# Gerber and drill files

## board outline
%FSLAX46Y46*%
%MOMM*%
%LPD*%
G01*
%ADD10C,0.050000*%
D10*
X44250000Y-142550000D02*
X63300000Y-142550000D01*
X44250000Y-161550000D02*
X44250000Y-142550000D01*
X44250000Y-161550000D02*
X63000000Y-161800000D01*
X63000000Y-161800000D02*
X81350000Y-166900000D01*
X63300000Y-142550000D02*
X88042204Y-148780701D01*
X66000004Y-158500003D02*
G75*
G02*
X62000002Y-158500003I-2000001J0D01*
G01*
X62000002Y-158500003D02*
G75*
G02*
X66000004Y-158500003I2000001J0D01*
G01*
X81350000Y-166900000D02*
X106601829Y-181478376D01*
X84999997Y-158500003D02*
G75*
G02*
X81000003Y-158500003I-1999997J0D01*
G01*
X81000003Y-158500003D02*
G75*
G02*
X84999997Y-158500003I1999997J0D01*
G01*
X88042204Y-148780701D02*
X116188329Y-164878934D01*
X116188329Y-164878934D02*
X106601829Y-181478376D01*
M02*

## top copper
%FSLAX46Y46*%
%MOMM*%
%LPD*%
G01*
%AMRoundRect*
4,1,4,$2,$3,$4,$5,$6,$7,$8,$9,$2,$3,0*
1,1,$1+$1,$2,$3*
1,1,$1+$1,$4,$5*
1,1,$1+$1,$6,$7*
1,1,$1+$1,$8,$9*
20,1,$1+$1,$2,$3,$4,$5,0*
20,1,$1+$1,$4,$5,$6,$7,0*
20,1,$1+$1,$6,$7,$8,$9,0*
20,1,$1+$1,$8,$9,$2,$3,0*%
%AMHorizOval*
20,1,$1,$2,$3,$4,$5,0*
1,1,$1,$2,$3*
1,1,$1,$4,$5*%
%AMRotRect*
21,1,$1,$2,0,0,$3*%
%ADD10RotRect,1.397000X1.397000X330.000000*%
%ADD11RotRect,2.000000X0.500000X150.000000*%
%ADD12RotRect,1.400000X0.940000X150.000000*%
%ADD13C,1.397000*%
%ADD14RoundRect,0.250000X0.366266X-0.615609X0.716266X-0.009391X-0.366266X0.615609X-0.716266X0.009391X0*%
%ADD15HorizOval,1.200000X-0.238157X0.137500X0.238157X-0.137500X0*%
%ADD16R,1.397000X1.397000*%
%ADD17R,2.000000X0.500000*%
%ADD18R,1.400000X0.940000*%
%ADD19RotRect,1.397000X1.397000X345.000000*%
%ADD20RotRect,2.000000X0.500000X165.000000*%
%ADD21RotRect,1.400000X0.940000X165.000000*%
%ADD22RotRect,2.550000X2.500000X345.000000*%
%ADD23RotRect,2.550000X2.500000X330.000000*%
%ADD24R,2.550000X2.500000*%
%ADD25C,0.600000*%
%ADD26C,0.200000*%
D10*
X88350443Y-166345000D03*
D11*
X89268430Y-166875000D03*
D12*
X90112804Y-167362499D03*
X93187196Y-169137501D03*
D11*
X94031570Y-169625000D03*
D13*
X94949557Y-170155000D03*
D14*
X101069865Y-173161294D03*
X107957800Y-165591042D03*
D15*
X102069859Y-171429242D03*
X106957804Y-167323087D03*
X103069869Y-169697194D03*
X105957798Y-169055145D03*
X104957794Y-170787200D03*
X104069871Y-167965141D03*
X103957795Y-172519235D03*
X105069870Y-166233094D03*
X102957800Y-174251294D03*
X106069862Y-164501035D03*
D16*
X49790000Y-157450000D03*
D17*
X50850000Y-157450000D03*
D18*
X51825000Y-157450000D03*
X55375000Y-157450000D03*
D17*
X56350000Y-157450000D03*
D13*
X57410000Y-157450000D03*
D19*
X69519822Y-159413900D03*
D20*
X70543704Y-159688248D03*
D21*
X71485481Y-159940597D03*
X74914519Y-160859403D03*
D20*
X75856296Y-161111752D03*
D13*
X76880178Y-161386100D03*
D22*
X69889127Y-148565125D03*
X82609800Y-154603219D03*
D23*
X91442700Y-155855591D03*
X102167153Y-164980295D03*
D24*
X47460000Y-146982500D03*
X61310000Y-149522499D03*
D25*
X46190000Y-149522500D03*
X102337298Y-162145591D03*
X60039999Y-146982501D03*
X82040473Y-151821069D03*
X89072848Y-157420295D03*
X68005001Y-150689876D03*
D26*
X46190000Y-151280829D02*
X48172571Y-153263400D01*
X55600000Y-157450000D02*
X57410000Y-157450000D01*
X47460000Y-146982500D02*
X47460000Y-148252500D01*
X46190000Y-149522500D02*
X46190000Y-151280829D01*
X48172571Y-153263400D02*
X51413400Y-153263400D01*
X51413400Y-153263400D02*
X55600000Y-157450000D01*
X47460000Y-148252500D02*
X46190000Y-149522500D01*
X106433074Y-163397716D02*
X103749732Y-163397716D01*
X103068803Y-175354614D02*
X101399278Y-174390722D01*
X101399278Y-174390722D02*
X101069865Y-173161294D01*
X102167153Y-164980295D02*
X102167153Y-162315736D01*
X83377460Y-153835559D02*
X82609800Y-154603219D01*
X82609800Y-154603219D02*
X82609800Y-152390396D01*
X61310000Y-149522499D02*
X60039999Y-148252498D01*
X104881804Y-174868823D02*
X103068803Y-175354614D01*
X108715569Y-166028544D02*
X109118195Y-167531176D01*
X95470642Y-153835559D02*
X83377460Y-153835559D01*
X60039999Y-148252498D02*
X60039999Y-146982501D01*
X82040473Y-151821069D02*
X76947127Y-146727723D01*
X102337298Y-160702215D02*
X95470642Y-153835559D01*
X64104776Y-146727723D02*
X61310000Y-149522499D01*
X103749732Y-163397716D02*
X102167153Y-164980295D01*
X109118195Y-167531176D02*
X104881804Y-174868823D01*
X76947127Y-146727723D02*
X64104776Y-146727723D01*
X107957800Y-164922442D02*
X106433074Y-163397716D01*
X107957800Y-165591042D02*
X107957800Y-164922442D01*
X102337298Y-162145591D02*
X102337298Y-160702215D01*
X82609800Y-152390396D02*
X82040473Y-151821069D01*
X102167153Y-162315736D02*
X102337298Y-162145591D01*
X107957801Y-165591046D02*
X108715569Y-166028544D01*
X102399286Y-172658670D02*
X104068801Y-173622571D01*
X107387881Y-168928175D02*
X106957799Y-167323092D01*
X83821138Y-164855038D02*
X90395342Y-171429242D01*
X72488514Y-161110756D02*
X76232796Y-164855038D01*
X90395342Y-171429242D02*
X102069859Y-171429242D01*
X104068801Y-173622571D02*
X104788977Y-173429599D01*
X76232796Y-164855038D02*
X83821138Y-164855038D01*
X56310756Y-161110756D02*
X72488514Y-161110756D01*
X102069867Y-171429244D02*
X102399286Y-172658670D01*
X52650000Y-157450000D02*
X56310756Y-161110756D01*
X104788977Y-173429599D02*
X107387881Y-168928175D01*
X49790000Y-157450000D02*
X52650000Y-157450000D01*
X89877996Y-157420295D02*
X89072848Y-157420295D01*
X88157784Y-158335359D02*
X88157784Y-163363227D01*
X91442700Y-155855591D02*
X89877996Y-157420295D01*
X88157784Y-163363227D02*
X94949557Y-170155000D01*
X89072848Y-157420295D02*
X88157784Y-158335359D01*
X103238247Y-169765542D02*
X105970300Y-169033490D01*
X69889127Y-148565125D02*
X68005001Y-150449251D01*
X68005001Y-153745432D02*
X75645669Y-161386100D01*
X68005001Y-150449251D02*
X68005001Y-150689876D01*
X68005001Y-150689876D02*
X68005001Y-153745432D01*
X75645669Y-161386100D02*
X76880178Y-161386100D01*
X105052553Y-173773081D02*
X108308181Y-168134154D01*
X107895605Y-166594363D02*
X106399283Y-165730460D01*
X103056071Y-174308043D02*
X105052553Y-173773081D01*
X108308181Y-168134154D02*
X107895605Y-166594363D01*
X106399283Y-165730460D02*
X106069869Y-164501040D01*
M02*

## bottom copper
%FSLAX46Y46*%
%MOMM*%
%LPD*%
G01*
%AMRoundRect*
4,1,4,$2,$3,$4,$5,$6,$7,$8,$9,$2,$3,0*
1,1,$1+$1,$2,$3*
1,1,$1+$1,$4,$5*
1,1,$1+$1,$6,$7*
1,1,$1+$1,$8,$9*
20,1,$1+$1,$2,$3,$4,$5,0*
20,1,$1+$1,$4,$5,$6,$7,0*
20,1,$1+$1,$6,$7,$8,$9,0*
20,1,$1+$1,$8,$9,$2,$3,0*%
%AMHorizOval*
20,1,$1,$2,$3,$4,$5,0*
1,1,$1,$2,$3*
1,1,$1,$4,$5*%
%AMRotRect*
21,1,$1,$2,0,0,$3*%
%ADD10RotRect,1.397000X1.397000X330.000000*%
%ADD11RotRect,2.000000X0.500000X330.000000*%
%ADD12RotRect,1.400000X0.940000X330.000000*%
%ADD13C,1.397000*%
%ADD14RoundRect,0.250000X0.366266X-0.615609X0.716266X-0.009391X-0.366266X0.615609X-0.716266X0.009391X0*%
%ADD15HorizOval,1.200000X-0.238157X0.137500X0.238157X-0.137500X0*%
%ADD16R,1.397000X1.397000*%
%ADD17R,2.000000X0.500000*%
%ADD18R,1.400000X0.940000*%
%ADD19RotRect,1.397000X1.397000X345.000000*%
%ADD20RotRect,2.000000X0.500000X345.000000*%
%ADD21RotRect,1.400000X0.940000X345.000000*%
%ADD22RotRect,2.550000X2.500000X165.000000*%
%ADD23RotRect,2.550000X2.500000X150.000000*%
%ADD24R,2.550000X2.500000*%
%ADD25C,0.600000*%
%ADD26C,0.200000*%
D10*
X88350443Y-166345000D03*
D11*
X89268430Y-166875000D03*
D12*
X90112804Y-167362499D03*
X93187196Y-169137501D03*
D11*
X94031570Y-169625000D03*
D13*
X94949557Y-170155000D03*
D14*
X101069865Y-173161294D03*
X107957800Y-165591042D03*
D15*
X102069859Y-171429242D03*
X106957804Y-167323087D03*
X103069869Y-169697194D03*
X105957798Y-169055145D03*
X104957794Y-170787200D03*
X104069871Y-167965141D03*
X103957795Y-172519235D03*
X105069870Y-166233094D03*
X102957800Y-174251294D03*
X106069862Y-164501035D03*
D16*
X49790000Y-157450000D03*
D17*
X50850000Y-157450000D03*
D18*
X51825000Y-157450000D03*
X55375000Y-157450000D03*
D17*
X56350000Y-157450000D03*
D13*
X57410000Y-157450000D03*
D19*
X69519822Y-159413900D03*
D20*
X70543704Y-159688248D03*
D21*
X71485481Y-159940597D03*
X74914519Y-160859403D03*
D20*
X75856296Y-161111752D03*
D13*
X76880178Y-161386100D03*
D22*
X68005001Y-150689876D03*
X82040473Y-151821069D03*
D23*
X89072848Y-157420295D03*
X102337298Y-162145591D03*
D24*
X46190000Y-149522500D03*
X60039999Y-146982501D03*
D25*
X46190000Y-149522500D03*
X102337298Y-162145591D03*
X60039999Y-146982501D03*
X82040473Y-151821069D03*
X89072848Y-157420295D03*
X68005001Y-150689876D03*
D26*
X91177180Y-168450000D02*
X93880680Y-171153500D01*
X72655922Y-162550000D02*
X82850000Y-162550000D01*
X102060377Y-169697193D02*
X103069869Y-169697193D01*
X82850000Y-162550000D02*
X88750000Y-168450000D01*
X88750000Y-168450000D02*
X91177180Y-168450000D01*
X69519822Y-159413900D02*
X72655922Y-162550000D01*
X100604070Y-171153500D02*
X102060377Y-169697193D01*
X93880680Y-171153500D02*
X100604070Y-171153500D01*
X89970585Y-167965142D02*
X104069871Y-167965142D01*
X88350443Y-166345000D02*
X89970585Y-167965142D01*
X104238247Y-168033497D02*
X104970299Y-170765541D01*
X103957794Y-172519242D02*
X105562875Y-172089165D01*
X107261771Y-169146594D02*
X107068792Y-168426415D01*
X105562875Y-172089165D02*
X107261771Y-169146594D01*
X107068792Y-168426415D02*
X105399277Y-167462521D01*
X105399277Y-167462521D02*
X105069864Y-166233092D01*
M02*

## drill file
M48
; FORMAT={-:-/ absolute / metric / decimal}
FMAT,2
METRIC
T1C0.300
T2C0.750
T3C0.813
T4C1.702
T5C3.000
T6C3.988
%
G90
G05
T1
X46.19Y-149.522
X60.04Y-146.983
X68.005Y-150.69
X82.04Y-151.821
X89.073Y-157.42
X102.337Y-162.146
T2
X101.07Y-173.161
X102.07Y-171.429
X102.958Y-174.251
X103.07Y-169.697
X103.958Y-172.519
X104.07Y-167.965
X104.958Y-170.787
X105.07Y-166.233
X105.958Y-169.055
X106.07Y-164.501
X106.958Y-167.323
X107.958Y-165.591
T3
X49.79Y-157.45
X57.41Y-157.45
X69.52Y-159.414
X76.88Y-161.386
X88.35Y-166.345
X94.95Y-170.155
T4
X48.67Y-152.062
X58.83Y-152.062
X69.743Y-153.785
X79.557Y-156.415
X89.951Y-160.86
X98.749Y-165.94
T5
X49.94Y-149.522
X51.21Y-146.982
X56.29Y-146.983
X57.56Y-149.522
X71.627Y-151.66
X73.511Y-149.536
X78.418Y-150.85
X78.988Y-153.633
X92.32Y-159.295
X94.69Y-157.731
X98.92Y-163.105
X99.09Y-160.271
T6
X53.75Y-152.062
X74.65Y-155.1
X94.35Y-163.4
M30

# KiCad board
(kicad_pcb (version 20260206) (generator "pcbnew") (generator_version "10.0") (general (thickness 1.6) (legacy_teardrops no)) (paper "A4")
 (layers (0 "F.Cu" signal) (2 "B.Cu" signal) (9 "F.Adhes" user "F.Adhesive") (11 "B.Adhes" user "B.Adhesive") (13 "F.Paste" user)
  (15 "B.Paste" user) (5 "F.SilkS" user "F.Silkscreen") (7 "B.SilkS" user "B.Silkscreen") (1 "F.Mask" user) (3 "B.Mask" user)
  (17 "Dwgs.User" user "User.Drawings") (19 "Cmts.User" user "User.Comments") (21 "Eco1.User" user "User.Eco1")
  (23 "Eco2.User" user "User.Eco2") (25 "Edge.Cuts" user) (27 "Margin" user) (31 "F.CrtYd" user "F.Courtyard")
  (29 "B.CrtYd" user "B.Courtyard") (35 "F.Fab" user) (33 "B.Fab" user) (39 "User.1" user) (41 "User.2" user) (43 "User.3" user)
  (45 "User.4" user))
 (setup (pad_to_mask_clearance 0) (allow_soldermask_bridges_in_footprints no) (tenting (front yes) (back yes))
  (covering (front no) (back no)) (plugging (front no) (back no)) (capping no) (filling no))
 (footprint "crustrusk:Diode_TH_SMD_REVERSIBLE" (layer "F.Cu") (at 91.65 168.25 -30)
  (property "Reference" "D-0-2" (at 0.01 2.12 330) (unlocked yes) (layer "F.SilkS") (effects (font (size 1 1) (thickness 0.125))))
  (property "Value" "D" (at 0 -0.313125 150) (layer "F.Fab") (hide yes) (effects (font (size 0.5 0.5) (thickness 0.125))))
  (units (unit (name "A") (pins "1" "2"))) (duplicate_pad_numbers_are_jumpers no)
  (pad "1" thru_hole rect (at -3.81 0 330) (size 1.397 1.397) (drill 0.8128) (layers "*.Cu" "*.Mask") (remove_unused_layers no)
   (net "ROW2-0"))
  (pad "1" smd rect (at -2.75 0 150) (size 2 0.5) (layers "F.Cu") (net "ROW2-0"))
  (pad "1" smd rect (at -2.75 0 330) (size 2 0.5) (layers "B.Cu") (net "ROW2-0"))
  (pad "1" smd rect (at -1.775001 0 150) (size 1.4 0.94) (layers "F.Cu" "F.Mask" "F.Paste") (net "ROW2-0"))
  (pad "1" smd rect (at -1.775001 0 330) (size 1.4 0.94) (layers "B.Cu" "B.Mask" "B.Paste") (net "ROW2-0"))
  (pad "2" smd rect (at 1.775001 0 150) (size 1.4 0.94) (layers "F.Cu" "F.Mask" "F.Paste") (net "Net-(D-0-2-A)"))
  (pad "2" smd rect (at 1.775001 0 330) (size 1.4 0.94) (layers "B.Cu" "B.Mask" "B.Paste") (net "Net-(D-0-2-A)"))
  (pad "2" smd rect (at 2.75 0 150) (size 2 0.5) (layers "F.Cu") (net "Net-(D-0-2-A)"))
  (pad "2" smd rect (at 2.75 0 330) (size 2 0.5) (layers "B.Cu") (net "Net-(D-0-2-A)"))
  (pad "2" thru_hole circle (at 3.81 0 330) (size 1.397 1.397) (drill 0.8128) (layers "*.Cu" "*.Mask") (remove_unused_layers no)
   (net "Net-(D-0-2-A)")))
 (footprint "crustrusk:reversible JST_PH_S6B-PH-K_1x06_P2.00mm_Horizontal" (layer "F.Cu") (at 101.069865 173.161294 60)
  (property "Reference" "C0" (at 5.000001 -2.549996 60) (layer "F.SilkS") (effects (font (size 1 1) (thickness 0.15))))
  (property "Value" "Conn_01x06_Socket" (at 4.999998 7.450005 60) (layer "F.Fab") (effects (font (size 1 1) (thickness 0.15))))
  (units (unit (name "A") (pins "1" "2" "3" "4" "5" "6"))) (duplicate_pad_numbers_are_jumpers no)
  (pad "1" thru_hole roundrect (at 0 0 60) (size 1.2 1.75) (drill 0.75) (layers "*.Cu" "*.Mask") (remove_unused_layers no)
   (roundrect_rratio 0.208333) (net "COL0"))
  (pad "1" thru_hole roundrect (at 9.999998 2.180001 60) (size 1.2 1.75) (drill 0.75) (layers "*.Cu" "*.Mask") (remove_unused_layers no)
   (roundrect_rratio 0.208333) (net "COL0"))
  (pad "2" thru_hole oval (at 1.999998 -0.000006 60) (size 1.2 1.75) (drill 0.75) (layers "*.Cu" "*.Mask") (remove_unused_layers no)
   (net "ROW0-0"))
  (pad "2" thru_hole oval (at 8.000005 2.180001 60) (size 1.2 1.75) (drill 0.75) (layers "*.Cu" "*.Mask") (remove_unused_layers no)
   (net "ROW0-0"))
  (pad "3" thru_hole oval (at 4.000001 0.000004 60) (size 1.2 1.75) (drill 0.75) (layers "*.Cu" "*.Mask") (remove_unused_layers no)
   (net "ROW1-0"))
  (pad "3" thru_hole oval (at 5.999996 2.18 60) (size 1.2 1.75) (drill 0.75) (layers "*.Cu" "*.Mask") (remove_unused_layers no)
   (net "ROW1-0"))
  (pad "4" thru_hole oval (at 3.99999 2.179998 60) (size 1.2 1.75) (drill 0.75) (layers "*.Cu" "*.Mask") (remove_unused_layers no)
   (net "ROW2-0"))
  (pad "4" thru_hole oval (at 6.000003 0.000005 60) (size 1.2 1.75) (drill 0.75) (layers "*.Cu" "*.Mask") (remove_unused_layers no)
   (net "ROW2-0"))
  (pad "5" thru_hole oval (at 2.000004 2.179991 60) (size 1.2 1.75) (drill 0.75) (layers "*.Cu" "*.Mask") (remove_unused_layers no)
   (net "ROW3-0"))
  (pad "5" thru_hole oval (at 8 0.000006 60) (size 1.2 1.75) (drill 0.75) (layers "*.Cu" "*.Mask") (remove_unused_layers no) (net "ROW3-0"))
  (pad "6" thru_hole oval (at 0 2.18 60) (size 1.2 1.75) (drill 0.75) (layers "*.Cu" "*.Mask") (remove_unused_layers no) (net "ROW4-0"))
  (pad "6" thru_hole oval (at 10.000003 -0.000005 60) (size 1.2 1.75) (drill 0.75) (layers "*.Cu" "*.Mask") (remove_unused_layers no)
   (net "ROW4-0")))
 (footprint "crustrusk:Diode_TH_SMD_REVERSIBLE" (layer "F.Cu") (at 53.6 157.45)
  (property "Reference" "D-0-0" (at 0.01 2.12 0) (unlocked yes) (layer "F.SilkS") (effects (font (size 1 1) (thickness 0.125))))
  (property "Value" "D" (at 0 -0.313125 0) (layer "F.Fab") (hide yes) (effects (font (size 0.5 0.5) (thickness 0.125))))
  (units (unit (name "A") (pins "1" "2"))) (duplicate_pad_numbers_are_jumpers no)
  (pad "1" thru_hole rect (at -3.81 0) (size 1.397 1.397) (drill 0.8128) (layers "*.Cu" "*.Mask") (remove_unused_layers no) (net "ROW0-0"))
  (pad "1" smd rect (at -2.75 0 180) (size 2 0.5) (layers "F.Cu") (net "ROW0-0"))
  (pad "1" smd rect (at -2.75 0) (size 2 0.5) (layers "B.Cu") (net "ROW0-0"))
  (pad "1" smd rect (at -1.775 0 180) (size 1.4 0.94) (layers "F.Cu" "F.Mask" "F.Paste") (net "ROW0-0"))
  (pad "1" smd rect (at -1.775 0) (size 1.4 0.94) (layers "B.Cu" "B.Mask" "B.Paste") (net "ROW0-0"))
  (pad "2" smd rect (at 1.775 0 180) (size 1.4 0.94) (layers "F.Cu" "F.Mask" "F.Paste") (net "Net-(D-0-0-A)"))
  (pad "2" smd rect (at 1.775 0) (size 1.4 0.94) (layers "B.Cu" "B.Mask" "B.Paste") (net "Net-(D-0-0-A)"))
  (pad "2" smd rect (at 2.75 0 180) (size 2 0.5) (layers "F.Cu") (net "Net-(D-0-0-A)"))
  (pad "2" smd rect (at 2.75 0) (size 2 0.5) (layers "B.Cu") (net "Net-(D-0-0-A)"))
  (pad "2" thru_hole circle (at 3.81 0) (size 1.397 1.397) (drill 0.8128) (layers "*.Cu" "*.Mask") (remove_unused_layers no)
   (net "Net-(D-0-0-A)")))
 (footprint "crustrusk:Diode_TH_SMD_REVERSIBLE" (layer "F.Cu") (at 73.2 160.4 -15)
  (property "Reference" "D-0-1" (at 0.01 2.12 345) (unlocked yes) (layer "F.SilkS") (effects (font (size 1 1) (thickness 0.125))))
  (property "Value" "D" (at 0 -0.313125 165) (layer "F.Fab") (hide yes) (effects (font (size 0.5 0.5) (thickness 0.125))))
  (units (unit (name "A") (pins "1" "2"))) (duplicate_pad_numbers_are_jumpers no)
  (pad "1" thru_hole rect (at -3.81 0.000001 345) (size 1.397 1.397) (drill 0.8128) (layers "*.Cu" "*.Mask") (remove_unused_layers no)
   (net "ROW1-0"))
  (pad "1" smd rect (at -2.75 0 165) (size 2 0.5) (layers "F.Cu") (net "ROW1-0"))
  (pad "1" smd rect (at -2.75 0 345) (size 2 0.5) (layers "B.Cu") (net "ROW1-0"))
  (pad "1" smd rect (at -1.775 0.000001 165) (size 1.4 0.94) (layers "F.Cu" "F.Mask" "F.Paste") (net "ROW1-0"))
  (pad "1" smd rect (at -1.775 0.000001 345) (size 1.4 0.94) (layers "B.Cu" "B.Mask" "B.Paste") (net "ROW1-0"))
  (pad "2" smd rect (at 1.775 -0.000001 165) (size 1.4 0.94) (layers "F.Cu" "F.Mask" "F.Paste") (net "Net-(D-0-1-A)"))
  (pad "2" smd rect (at 1.775 -0.000001 345) (size 1.4 0.94) (layers "B.Cu" "B.Mask" "B.Paste") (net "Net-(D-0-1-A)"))
  (pad "2" smd rect (at 2.75 0 165) (size 2 0.5) (layers "F.Cu") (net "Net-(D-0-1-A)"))
  (pad "2" smd rect (at 2.75 0 345) (size 2 0.5) (layers "B.Cu") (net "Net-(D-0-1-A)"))
  (pad "2" thru_hole circle (at 3.81 -0.000001 345) (size 1.397 1.397) (drill 0.8128) (layers "*.Cu" "*.Mask") (remove_unused_layers no)
   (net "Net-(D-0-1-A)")))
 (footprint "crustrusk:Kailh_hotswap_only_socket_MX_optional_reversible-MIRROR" (layer "B.Cu") (at 74.65 155.1 165)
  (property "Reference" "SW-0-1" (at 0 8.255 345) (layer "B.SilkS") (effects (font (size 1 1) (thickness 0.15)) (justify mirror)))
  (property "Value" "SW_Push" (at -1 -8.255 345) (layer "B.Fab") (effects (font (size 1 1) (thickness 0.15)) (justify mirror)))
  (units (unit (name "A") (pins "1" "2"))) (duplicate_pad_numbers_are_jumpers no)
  (pad "" np_thru_hole circle (at -5.08 0 165) (size 1.7018 1.7018) (drill 1.7018) (layers "*.Cu" "*.Mask"))
  (pad "" np_thru_hole circle (at -3.81 2.54 345) (size 3 3) (drill 3) (layers "*.Cu" "*.Mask"))
  (pad "" np_thru_hole circle (at -2.54 5.079998 165) (size 3 3) (drill 3) (layers "*.Cu" "*.Mask"))
  (pad "" np_thru_hole circle (at 0 0 165) (size 3.9878 3.9878) (drill 3.9878) (layers "*.Cu" "*.Mask"))
  (pad "" np_thru_hole circle (at 2.540002 5.080001 345) (size 3 3) (drill 3) (layers "*.Cu" "*.Mask"))
  (pad "" np_thru_hole circle (at 3.81 2.54 165) (size 3 3) (drill 3) (layers "*.Cu" "*.Mask"))
  (pad "" np_thru_hole circle (at 5.08 0 165) (size 1.7018 1.7018) (drill 1.7018) (layers "*.Cu" "*.Mask"))
  (pad "1" smd rect (at 6.29 5.08 345) (size 2.55 2.5) (layers "F.Cu" "F.Mask" "F.Paste") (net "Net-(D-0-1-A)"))
  (pad "1" smd rect (at 7.56 2.54 165) (size 2.55 2.5) (layers "B.Cu" "B.Mask" "B.Paste") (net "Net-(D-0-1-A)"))
  (pad "2" smd rect (at -7.56 2.540001 345) (size 2.55 2.5) (layers "F.Cu" "F.Mask" "F.Paste") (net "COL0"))
  (pad "2" smd rect (at -6.289999 5.079999 165) (size 2.55 2.5) (layers "B.Cu" "B.Mask" "B.Paste") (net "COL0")))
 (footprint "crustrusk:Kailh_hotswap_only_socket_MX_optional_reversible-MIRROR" (layer "B.Cu") (at 94.35 163.4 150)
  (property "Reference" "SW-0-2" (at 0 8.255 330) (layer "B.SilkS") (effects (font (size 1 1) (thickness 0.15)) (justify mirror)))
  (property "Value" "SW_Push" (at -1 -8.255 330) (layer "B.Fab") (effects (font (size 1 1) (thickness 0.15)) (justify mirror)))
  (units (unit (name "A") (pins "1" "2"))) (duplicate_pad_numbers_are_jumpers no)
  (pad "" np_thru_hole circle (at -5.08 0 150) (size 1.7018 1.7018) (drill 1.7018) (layers "*.Cu" "*.Mask"))
  (pad "" np_thru_hole circle (at -3.81 2.540001 330) (size 3 3) (drill 3) (layers "*.Cu" "*.Mask"))
  (pad "" np_thru_hole circle (at -2.540001 5.079998 150) (size 3 3) (drill 3) (layers "*.Cu" "*.Mask"))
  (pad "" np_thru_hole circle (at 0 0 150) (size 3.9878 3.9878) (drill 3.9878) (layers "*.Cu" "*.Mask"))
  (pad "" np_thru_hole circle (at 2.540002 5.080001 330) (size 3 3) (drill 3) (layers "*.Cu" "*.Mask"))
  (pad "" np_thru_hole circle (at 3.81 2.54 150) (size 3 3) (drill 3) (layers "*.Cu" "*.Mask"))
  (pad "" np_thru_hole circle (at 5.08 0 150) (size 1.7018 1.7018) (drill 1.7018) (layers "*.Cu" "*.Mask"))
  (pad "1" smd rect (at 6.29 5.08 330) (size 2.55 2.5) (layers "F.Cu" "F.Mask" "F.Paste") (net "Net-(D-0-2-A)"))
  (pad "1" smd rect (at 7.56 2.54 150) (size 2.55 2.5) (layers "B.Cu" "B.Mask" "B.Paste") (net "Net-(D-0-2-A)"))
  (pad "2" smd rect (at -7.560001 2.540001 330) (size 2.55 2.5) (layers "F.Cu" "F.Mask" "F.Paste") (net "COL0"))
  (pad "2" smd rect (at -6.289998 5.079999 150) (size 2.55 2.5) (layers "B.Cu" "B.Mask" "B.Paste") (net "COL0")))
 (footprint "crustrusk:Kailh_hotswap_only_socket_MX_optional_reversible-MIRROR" (layer "B.Cu") (at 53.75 152.0625 180)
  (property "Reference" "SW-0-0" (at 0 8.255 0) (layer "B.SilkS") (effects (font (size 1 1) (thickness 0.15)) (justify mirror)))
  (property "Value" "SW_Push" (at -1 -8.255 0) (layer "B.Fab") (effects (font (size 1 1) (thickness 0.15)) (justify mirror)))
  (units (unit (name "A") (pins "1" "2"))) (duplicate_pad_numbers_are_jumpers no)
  (pad "" np_thru_hole circle (at -5.08 0 180) (size 1.7018 1.7018) (drill 1.7018) (layers "*.Cu" "*.Mask"))
  (pad "" np_thru_hole circle (at -3.81 2.54) (size 3 3) (drill 3) (layers "*.Cu" "*.Mask"))
  (pad "" np_thru_hole circle (at -2.54 5.079998 180) (size 3 3) (drill 3) (layers "*.Cu" "*.Mask"))
  (pad "" np_thru_hole circle (at 0 0 180) (size 3.9878 3.9878) (drill 3.9878) (layers "*.Cu" "*.Mask"))
  (pad "" np_thru_hole circle (at 2.540002 5.080001) (size 3 3) (drill 3) (layers "*.Cu" "*.Mask"))
  (pad "" np_thru_hole circle (at 3.81 2.54 180) (size 3 3) (drill 3) (layers "*.Cu" "*.Mask"))
  (pad "" np_thru_hole circle (at 5.08 0 180) (size 1.7018 1.7018) (drill 1.7018) (layers "*.Cu" "*.Mask"))
  (pad "1" smd rect (at 6.29 5.08) (size 2.55 2.5) (layers "F.Cu" "F.Mask" "F.Paste") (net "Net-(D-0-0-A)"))
  (pad "1" smd rect (at 7.56 2.54 180) (size 2.55 2.5) (layers "B.Cu" "B.Mask" "B.Paste") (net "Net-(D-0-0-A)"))
  (pad "2" smd rect (at -7.56 2.540001) (size 2.55 2.5) (layers "F.Cu" "F.Mask" "F.Paste") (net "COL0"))
  (pad "2" smd rect (at -6.289999 5.079999 180) (size 2.55 2.5) (layers "B.Cu" "B.Mask" "B.Paste") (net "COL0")))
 (gr_line (start 44.25 142.55) (end 63.3 142.55) (stroke (width 0.05) (type default)) (layer "Edge.Cuts"))
 (gr_line (start 44.25 161.55) (end 44.25 142.55) (stroke (width 0.05) (type default)) (layer "Edge.Cuts"))
 (gr_line (start 44.25 161.55) (end 63 161.8) (stroke (width 0.05) (type default)) (layer "Edge.Cuts"))
 (gr_line (start 63 161.8) (end 81.35 166.9) (stroke (width 0.05) (type default)) (layer "Edge.Cuts"))
 (gr_line (start 63.3 142.55) (end 88.042204 148.780701) (stroke (width 0.05) (type default)) (layer "Edge.Cuts"))
 (gr_circle (center 64.000003 158.500003) (end 62.000002 158.500003) (stroke (width 0.05) (type default)) (fill no) (layer "Edge.Cuts"))
 (gr_line (start 81.35 166.9) (end 106.601829 181.478376) (stroke (width 0.05) (type default)) (layer "Edge.Cuts"))
 (gr_circle (center 83 158.500003) (end 81.000003 158.500003) (stroke (width 0.05) (type default)) (fill no) (layer "Edge.Cuts"))
 (gr_line (start 88.042204 148.780701) (end 116.188329 164.878934) (stroke (width 0.05) (type default)) (layer "Edge.Cuts"))
 (gr_line (start 116.188329 164.878934) (end 106.601829 181.478376) (stroke (width 0.05) (type default)) (layer "Edge.Cuts"))
 (segment (start 46.19 151.280829) (end 48.172571 153.2634) (width 0.2) (layer "F.Cu") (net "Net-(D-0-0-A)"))
 (segment (start 55.6 157.45) (end 57.41 157.45) (width 0.2) (layer "F.Cu") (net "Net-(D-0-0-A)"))
 (segment (start 47.46 146.9825) (end 47.46 148.2525) (width 0.2) (layer "F.Cu") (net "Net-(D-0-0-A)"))
 (segment (start 46.19 149.5225) (end 46.19 151.280829) (width 0.2) (layer "F.Cu") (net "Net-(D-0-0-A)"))
 (segment (start 48.172571 153.2634) (end 51.4134 153.2634) (width 0.2) (layer "F.Cu") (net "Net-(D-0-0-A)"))
 (segment (start 51.4134 153.2634) (end 55.6 157.45) (width 0.2) (layer "F.Cu") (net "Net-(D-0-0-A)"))
 (segment (start 47.46 148.2525) (end 46.19 149.5225) (width 0.2) (layer "F.Cu") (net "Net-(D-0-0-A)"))
 (via (at 46.19 149.5225) (size 0.6) (drill 0.3) (layers "F.Cu" "B.Cu") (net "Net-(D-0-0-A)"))
 (segment (start 106.433074 163.397716) (end 103.749732 163.397716) (width 0.2) (layer "F.Cu") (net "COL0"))
 (segment (start 103.068803 175.354614) (end 101.399278 174.390722) (width 0.2) (layer "F.Cu") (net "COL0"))
 (segment (start 101.399278 174.390722) (end 101.069865 173.161294) (width 0.2) (layer "F.Cu") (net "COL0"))
 (segment (start 102.167153 164.980295) (end 102.167153 162.315736) (width 0.2) (layer "F.Cu") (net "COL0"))
 (segment (start 83.37746 153.835559) (end 82.6098 154.603219) (width 0.2) (layer "F.Cu") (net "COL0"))
 (segment (start 82.6098 154.603219) (end 82.6098 152.390396) (width 0.2) (layer "F.Cu") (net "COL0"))
 (segment (start 61.31 149.522499) (end 60.039999 148.252498) (width 0.2) (layer "F.Cu") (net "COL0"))
 (segment (start 104.881804 174.868823) (end 103.068803 175.354614) (width 0.2) (layer "F.Cu") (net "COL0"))
 (segment (start 108.715569 166.028544) (end 109.118195 167.531176) (width 0.2) (layer "F.Cu") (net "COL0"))
 (segment (start 95.470642 153.835559) (end 83.37746 153.835559) (width 0.2) (layer "F.Cu") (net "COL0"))
 (segment (start 60.039999 148.252498) (end 60.039999 146.982501) (width 0.2) (layer "F.Cu") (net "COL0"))
 (segment (start 82.040473 151.821069) (end 76.947127 146.727723) (width 0.2) (layer "F.Cu") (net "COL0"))
 (segment (start 102.337298 160.702215) (end 95.470642 153.835559) (width 0.2) (layer "F.Cu") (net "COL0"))
 (segment (start 64.104776 146.727723) (end 61.31 149.522499) (width 0.2) (layer "F.Cu") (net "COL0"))
 (segment (start 103.749732 163.397716) (end 102.167153 164.980295) (width 0.2) (layer "F.Cu") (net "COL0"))
 (segment (start 109.118195 167.531176) (end 104.881804 174.868823) (width 0.2) (layer "F.Cu") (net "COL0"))
 (segment (start 76.947127 146.727723) (end 64.104776 146.727723) (width 0.2) (layer "F.Cu") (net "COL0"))
 (segment (start 107.9578 164.922442) (end 106.433074 163.397716) (width 0.2) (layer "F.Cu") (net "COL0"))
 (segment (start 107.9578 165.591042) (end 107.9578 164.922442) (width 0.2) (layer "F.Cu") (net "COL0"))
 (segment (start 102.337298 162.145591) (end 102.337298 160.702215) (width 0.2) (layer "F.Cu") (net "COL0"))
 (segment (start 82.6098 152.390396) (end 82.040473 151.821069) (width 0.2) (layer "F.Cu") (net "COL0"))
 (segment (start 102.167153 162.315736) (end 102.337298 162.145591) (width 0.2) (layer "F.Cu") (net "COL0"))
 (segment (start 107.957801 165.591046) (end 108.715569 166.028544) (width 0.2) (layer "F.Cu") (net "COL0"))
 (via (at 102.337298 162.145591) (size 0.6) (drill 0.3) (layers "F.Cu" "B.Cu") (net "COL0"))
 (via (at 60.039999 146.982501) (size 0.6) (drill 0.3) (layers "F.Cu" "B.Cu") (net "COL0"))
 (via (at 82.040473 151.821069) (size 0.6) (drill 0.3) (layers "F.Cu" "B.Cu") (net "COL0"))
 (segment (start 102.399286 172.65867) (end 104.068801 173.622571) (width 0.2) (layer "F.Cu") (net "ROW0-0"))
 (segment (start 107.387881 168.928175) (end 106.957799 167.323092) (width 0.2) (layer "F.Cu") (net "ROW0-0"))
 (segment (start 83.821138 164.855038) (end 90.395342 171.429242) (width 0.2) (layer "F.Cu") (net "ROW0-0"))
 (segment (start 72.488514 161.110756) (end 76.232796 164.855038) (width 0.2) (layer "F.Cu") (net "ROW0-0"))
 (segment (start 90.395342 171.429242) (end 102.069859 171.429242) (width 0.2) (layer "F.Cu") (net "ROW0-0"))
 (segment (start 104.068801 173.622571) (end 104.788977 173.429599) (width 0.2) (layer "F.Cu") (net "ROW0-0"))
 (segment (start 76.232796 164.855038) (end 83.821138 164.855038) (width 0.2) (layer "F.Cu") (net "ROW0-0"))
 (segment (start 56.310756 161.110756) (end 72.488514 161.110756) (width 0.2) (layer "F.Cu") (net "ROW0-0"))
 (segment (start 102.069867 171.429244) (end 102.399286 172.65867) (width 0.2) (layer "F.Cu") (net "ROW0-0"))
 (segment (start 52.65 157.45) (end 56.310756 161.110756) (width 0.2) (layer "F.Cu") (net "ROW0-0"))
 (segment (start 104.788977 173.429599) (end 107.387881 168.928175) (width 0.2) (layer "F.Cu") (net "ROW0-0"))
 (segment (start 49.79 157.45) (end 52.65 157.45) (width 0.2) (layer "F.Cu") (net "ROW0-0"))
 (segment (start 89.877996 157.420295) (end 89.072848 157.420295) (width 0.2) (layer "F.Cu") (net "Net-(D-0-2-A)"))
 (segment (start 88.157784 158.335359) (end 88.157784 163.363227) (width 0.2) (layer "F.Cu") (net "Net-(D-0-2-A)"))
 (segment (start 91.4427 155.855591) (end 89.877996 157.420295) (width 0.2) (layer "F.Cu") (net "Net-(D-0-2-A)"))
 (segment (start 88.157784 163.363227) (end 94.949557 170.155) (width 0.2) (layer "F.Cu") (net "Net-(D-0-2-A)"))
 (segment (start 89.072848 157.420295) (end 88.157784 158.335359) (width 0.2) (layer "F.Cu") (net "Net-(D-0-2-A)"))
 (via (at 89.072848 157.420295) (size 0.6) (drill 0.3) (layers "F.Cu" "B.Cu") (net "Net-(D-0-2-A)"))
 (segment (start 103.238247 169.765542) (end 105.9703 169.03349) (width 0.2) (layer "F.Cu") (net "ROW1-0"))
 (segment (start 91.17718 168.45) (end 93.88068 171.1535) (width 0.2) (layer "B.Cu") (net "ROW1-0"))
 (segment (start 72.655922 162.55) (end 82.85 162.55) (width 0.2) (layer "B.Cu") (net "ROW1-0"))
 (segment (start 102.060377 169.697193) (end 103.069869 169.697193) (width 0.2) (layer "B.Cu") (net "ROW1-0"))
 (segment (start 82.85 162.55) (end 88.75 168.45) (width 0.2) (layer "B.Cu") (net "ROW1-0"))
 (segment (start 88.75 168.45) (end 91.17718 168.45) (width 0.2) (layer "B.Cu") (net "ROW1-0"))
 (segment (start 69.519822 159.4139) (end 72.655922 162.55) (width 0.2) (layer "B.Cu") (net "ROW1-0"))
 (segment (start 100.60407 171.1535) (end 102.060377 169.697193) (width 0.2) (layer "B.Cu") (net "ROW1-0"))
 (segment (start 93.88068 171.1535) (end 100.60407 171.1535) (width 0.2) (layer "B.Cu") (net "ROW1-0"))
 (segment (start 69.889127 148.565125) (end 68.005001 150.449251) (width 0.2) (layer "F.Cu") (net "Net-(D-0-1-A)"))
 (segment (start 68.005001 153.745432) (end 75.645669 161.3861) (width 0.2) (layer "F.Cu") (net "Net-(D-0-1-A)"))
 (segment (start 68.005001 150.449251) (end 68.005001 150.689876) (width 0.2) (layer "F.Cu") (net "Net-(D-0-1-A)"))
 (segment (start 68.005001 150.689876) (end 68.005001 153.745432) (width 0.2) (layer "F.Cu") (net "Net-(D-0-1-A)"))
 (segment (start 75.645669 161.3861) (end 76.880178 161.3861) (width 0.2) (layer "F.Cu") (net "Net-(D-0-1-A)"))
 (via (at 68.005001 150.689876) (size 0.6) (drill 0.3) (layers "F.Cu" "B.Cu") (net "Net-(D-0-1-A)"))
 (segment (start 89.970585 167.965142) (end 104.069871 167.965142) (width 0.2) (layer "B.Cu") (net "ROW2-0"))
 (segment (start 88.350443 166.345) (end 89.970585 167.965142) (width 0.2) (layer "B.Cu") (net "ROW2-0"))
 (segment (start 104.238247 168.033497) (end 104.970299 170.765541) (width 0.2) (layer "B.Cu") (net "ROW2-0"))
 (segment (start 103.957794 172.519242) (end 105.562875 172.089165) (width 0.2) (layer "B.Cu") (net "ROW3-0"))
 (segment (start 107.261771 169.146594) (end 107.068792 168.426415) (width 0.2) (layer "B.Cu") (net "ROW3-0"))
 (segment (start 105.562875 172.089165) (end 107.261771 169.146594) (width 0.2) (layer "B.Cu") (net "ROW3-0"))
 (segment (start 107.068792 168.426415) (end 105.399277 167.462521) (width 0.2) (layer "B.Cu") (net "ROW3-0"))
 (segment (start 105.399277 167.462521) (end 105.069864 166.233092) (width 0.2) (layer "B.Cu") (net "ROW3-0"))
 (segment (start 105.052553 173.773081) (end 108.308181 168.134154) (width 0.2) (layer "F.Cu") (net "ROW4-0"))
 (segment (start 107.895605 166.594363) (end 106.399283 165.73046) (width 0.2) (layer "F.Cu") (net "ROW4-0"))
 (segment (start 103.056071 174.308043) (end 105.052553 173.773081) (width 0.2) (layer "F.Cu") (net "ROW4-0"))
 (segment (start 108.308181 168.134154) (end 107.895605 166.594363) (width 0.2) (layer "F.Cu") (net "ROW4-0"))
 (segment (start 106.399283 165.73046) (end 106.069869 164.50104) (width 0.2) (layer "F.Cu") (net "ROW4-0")))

